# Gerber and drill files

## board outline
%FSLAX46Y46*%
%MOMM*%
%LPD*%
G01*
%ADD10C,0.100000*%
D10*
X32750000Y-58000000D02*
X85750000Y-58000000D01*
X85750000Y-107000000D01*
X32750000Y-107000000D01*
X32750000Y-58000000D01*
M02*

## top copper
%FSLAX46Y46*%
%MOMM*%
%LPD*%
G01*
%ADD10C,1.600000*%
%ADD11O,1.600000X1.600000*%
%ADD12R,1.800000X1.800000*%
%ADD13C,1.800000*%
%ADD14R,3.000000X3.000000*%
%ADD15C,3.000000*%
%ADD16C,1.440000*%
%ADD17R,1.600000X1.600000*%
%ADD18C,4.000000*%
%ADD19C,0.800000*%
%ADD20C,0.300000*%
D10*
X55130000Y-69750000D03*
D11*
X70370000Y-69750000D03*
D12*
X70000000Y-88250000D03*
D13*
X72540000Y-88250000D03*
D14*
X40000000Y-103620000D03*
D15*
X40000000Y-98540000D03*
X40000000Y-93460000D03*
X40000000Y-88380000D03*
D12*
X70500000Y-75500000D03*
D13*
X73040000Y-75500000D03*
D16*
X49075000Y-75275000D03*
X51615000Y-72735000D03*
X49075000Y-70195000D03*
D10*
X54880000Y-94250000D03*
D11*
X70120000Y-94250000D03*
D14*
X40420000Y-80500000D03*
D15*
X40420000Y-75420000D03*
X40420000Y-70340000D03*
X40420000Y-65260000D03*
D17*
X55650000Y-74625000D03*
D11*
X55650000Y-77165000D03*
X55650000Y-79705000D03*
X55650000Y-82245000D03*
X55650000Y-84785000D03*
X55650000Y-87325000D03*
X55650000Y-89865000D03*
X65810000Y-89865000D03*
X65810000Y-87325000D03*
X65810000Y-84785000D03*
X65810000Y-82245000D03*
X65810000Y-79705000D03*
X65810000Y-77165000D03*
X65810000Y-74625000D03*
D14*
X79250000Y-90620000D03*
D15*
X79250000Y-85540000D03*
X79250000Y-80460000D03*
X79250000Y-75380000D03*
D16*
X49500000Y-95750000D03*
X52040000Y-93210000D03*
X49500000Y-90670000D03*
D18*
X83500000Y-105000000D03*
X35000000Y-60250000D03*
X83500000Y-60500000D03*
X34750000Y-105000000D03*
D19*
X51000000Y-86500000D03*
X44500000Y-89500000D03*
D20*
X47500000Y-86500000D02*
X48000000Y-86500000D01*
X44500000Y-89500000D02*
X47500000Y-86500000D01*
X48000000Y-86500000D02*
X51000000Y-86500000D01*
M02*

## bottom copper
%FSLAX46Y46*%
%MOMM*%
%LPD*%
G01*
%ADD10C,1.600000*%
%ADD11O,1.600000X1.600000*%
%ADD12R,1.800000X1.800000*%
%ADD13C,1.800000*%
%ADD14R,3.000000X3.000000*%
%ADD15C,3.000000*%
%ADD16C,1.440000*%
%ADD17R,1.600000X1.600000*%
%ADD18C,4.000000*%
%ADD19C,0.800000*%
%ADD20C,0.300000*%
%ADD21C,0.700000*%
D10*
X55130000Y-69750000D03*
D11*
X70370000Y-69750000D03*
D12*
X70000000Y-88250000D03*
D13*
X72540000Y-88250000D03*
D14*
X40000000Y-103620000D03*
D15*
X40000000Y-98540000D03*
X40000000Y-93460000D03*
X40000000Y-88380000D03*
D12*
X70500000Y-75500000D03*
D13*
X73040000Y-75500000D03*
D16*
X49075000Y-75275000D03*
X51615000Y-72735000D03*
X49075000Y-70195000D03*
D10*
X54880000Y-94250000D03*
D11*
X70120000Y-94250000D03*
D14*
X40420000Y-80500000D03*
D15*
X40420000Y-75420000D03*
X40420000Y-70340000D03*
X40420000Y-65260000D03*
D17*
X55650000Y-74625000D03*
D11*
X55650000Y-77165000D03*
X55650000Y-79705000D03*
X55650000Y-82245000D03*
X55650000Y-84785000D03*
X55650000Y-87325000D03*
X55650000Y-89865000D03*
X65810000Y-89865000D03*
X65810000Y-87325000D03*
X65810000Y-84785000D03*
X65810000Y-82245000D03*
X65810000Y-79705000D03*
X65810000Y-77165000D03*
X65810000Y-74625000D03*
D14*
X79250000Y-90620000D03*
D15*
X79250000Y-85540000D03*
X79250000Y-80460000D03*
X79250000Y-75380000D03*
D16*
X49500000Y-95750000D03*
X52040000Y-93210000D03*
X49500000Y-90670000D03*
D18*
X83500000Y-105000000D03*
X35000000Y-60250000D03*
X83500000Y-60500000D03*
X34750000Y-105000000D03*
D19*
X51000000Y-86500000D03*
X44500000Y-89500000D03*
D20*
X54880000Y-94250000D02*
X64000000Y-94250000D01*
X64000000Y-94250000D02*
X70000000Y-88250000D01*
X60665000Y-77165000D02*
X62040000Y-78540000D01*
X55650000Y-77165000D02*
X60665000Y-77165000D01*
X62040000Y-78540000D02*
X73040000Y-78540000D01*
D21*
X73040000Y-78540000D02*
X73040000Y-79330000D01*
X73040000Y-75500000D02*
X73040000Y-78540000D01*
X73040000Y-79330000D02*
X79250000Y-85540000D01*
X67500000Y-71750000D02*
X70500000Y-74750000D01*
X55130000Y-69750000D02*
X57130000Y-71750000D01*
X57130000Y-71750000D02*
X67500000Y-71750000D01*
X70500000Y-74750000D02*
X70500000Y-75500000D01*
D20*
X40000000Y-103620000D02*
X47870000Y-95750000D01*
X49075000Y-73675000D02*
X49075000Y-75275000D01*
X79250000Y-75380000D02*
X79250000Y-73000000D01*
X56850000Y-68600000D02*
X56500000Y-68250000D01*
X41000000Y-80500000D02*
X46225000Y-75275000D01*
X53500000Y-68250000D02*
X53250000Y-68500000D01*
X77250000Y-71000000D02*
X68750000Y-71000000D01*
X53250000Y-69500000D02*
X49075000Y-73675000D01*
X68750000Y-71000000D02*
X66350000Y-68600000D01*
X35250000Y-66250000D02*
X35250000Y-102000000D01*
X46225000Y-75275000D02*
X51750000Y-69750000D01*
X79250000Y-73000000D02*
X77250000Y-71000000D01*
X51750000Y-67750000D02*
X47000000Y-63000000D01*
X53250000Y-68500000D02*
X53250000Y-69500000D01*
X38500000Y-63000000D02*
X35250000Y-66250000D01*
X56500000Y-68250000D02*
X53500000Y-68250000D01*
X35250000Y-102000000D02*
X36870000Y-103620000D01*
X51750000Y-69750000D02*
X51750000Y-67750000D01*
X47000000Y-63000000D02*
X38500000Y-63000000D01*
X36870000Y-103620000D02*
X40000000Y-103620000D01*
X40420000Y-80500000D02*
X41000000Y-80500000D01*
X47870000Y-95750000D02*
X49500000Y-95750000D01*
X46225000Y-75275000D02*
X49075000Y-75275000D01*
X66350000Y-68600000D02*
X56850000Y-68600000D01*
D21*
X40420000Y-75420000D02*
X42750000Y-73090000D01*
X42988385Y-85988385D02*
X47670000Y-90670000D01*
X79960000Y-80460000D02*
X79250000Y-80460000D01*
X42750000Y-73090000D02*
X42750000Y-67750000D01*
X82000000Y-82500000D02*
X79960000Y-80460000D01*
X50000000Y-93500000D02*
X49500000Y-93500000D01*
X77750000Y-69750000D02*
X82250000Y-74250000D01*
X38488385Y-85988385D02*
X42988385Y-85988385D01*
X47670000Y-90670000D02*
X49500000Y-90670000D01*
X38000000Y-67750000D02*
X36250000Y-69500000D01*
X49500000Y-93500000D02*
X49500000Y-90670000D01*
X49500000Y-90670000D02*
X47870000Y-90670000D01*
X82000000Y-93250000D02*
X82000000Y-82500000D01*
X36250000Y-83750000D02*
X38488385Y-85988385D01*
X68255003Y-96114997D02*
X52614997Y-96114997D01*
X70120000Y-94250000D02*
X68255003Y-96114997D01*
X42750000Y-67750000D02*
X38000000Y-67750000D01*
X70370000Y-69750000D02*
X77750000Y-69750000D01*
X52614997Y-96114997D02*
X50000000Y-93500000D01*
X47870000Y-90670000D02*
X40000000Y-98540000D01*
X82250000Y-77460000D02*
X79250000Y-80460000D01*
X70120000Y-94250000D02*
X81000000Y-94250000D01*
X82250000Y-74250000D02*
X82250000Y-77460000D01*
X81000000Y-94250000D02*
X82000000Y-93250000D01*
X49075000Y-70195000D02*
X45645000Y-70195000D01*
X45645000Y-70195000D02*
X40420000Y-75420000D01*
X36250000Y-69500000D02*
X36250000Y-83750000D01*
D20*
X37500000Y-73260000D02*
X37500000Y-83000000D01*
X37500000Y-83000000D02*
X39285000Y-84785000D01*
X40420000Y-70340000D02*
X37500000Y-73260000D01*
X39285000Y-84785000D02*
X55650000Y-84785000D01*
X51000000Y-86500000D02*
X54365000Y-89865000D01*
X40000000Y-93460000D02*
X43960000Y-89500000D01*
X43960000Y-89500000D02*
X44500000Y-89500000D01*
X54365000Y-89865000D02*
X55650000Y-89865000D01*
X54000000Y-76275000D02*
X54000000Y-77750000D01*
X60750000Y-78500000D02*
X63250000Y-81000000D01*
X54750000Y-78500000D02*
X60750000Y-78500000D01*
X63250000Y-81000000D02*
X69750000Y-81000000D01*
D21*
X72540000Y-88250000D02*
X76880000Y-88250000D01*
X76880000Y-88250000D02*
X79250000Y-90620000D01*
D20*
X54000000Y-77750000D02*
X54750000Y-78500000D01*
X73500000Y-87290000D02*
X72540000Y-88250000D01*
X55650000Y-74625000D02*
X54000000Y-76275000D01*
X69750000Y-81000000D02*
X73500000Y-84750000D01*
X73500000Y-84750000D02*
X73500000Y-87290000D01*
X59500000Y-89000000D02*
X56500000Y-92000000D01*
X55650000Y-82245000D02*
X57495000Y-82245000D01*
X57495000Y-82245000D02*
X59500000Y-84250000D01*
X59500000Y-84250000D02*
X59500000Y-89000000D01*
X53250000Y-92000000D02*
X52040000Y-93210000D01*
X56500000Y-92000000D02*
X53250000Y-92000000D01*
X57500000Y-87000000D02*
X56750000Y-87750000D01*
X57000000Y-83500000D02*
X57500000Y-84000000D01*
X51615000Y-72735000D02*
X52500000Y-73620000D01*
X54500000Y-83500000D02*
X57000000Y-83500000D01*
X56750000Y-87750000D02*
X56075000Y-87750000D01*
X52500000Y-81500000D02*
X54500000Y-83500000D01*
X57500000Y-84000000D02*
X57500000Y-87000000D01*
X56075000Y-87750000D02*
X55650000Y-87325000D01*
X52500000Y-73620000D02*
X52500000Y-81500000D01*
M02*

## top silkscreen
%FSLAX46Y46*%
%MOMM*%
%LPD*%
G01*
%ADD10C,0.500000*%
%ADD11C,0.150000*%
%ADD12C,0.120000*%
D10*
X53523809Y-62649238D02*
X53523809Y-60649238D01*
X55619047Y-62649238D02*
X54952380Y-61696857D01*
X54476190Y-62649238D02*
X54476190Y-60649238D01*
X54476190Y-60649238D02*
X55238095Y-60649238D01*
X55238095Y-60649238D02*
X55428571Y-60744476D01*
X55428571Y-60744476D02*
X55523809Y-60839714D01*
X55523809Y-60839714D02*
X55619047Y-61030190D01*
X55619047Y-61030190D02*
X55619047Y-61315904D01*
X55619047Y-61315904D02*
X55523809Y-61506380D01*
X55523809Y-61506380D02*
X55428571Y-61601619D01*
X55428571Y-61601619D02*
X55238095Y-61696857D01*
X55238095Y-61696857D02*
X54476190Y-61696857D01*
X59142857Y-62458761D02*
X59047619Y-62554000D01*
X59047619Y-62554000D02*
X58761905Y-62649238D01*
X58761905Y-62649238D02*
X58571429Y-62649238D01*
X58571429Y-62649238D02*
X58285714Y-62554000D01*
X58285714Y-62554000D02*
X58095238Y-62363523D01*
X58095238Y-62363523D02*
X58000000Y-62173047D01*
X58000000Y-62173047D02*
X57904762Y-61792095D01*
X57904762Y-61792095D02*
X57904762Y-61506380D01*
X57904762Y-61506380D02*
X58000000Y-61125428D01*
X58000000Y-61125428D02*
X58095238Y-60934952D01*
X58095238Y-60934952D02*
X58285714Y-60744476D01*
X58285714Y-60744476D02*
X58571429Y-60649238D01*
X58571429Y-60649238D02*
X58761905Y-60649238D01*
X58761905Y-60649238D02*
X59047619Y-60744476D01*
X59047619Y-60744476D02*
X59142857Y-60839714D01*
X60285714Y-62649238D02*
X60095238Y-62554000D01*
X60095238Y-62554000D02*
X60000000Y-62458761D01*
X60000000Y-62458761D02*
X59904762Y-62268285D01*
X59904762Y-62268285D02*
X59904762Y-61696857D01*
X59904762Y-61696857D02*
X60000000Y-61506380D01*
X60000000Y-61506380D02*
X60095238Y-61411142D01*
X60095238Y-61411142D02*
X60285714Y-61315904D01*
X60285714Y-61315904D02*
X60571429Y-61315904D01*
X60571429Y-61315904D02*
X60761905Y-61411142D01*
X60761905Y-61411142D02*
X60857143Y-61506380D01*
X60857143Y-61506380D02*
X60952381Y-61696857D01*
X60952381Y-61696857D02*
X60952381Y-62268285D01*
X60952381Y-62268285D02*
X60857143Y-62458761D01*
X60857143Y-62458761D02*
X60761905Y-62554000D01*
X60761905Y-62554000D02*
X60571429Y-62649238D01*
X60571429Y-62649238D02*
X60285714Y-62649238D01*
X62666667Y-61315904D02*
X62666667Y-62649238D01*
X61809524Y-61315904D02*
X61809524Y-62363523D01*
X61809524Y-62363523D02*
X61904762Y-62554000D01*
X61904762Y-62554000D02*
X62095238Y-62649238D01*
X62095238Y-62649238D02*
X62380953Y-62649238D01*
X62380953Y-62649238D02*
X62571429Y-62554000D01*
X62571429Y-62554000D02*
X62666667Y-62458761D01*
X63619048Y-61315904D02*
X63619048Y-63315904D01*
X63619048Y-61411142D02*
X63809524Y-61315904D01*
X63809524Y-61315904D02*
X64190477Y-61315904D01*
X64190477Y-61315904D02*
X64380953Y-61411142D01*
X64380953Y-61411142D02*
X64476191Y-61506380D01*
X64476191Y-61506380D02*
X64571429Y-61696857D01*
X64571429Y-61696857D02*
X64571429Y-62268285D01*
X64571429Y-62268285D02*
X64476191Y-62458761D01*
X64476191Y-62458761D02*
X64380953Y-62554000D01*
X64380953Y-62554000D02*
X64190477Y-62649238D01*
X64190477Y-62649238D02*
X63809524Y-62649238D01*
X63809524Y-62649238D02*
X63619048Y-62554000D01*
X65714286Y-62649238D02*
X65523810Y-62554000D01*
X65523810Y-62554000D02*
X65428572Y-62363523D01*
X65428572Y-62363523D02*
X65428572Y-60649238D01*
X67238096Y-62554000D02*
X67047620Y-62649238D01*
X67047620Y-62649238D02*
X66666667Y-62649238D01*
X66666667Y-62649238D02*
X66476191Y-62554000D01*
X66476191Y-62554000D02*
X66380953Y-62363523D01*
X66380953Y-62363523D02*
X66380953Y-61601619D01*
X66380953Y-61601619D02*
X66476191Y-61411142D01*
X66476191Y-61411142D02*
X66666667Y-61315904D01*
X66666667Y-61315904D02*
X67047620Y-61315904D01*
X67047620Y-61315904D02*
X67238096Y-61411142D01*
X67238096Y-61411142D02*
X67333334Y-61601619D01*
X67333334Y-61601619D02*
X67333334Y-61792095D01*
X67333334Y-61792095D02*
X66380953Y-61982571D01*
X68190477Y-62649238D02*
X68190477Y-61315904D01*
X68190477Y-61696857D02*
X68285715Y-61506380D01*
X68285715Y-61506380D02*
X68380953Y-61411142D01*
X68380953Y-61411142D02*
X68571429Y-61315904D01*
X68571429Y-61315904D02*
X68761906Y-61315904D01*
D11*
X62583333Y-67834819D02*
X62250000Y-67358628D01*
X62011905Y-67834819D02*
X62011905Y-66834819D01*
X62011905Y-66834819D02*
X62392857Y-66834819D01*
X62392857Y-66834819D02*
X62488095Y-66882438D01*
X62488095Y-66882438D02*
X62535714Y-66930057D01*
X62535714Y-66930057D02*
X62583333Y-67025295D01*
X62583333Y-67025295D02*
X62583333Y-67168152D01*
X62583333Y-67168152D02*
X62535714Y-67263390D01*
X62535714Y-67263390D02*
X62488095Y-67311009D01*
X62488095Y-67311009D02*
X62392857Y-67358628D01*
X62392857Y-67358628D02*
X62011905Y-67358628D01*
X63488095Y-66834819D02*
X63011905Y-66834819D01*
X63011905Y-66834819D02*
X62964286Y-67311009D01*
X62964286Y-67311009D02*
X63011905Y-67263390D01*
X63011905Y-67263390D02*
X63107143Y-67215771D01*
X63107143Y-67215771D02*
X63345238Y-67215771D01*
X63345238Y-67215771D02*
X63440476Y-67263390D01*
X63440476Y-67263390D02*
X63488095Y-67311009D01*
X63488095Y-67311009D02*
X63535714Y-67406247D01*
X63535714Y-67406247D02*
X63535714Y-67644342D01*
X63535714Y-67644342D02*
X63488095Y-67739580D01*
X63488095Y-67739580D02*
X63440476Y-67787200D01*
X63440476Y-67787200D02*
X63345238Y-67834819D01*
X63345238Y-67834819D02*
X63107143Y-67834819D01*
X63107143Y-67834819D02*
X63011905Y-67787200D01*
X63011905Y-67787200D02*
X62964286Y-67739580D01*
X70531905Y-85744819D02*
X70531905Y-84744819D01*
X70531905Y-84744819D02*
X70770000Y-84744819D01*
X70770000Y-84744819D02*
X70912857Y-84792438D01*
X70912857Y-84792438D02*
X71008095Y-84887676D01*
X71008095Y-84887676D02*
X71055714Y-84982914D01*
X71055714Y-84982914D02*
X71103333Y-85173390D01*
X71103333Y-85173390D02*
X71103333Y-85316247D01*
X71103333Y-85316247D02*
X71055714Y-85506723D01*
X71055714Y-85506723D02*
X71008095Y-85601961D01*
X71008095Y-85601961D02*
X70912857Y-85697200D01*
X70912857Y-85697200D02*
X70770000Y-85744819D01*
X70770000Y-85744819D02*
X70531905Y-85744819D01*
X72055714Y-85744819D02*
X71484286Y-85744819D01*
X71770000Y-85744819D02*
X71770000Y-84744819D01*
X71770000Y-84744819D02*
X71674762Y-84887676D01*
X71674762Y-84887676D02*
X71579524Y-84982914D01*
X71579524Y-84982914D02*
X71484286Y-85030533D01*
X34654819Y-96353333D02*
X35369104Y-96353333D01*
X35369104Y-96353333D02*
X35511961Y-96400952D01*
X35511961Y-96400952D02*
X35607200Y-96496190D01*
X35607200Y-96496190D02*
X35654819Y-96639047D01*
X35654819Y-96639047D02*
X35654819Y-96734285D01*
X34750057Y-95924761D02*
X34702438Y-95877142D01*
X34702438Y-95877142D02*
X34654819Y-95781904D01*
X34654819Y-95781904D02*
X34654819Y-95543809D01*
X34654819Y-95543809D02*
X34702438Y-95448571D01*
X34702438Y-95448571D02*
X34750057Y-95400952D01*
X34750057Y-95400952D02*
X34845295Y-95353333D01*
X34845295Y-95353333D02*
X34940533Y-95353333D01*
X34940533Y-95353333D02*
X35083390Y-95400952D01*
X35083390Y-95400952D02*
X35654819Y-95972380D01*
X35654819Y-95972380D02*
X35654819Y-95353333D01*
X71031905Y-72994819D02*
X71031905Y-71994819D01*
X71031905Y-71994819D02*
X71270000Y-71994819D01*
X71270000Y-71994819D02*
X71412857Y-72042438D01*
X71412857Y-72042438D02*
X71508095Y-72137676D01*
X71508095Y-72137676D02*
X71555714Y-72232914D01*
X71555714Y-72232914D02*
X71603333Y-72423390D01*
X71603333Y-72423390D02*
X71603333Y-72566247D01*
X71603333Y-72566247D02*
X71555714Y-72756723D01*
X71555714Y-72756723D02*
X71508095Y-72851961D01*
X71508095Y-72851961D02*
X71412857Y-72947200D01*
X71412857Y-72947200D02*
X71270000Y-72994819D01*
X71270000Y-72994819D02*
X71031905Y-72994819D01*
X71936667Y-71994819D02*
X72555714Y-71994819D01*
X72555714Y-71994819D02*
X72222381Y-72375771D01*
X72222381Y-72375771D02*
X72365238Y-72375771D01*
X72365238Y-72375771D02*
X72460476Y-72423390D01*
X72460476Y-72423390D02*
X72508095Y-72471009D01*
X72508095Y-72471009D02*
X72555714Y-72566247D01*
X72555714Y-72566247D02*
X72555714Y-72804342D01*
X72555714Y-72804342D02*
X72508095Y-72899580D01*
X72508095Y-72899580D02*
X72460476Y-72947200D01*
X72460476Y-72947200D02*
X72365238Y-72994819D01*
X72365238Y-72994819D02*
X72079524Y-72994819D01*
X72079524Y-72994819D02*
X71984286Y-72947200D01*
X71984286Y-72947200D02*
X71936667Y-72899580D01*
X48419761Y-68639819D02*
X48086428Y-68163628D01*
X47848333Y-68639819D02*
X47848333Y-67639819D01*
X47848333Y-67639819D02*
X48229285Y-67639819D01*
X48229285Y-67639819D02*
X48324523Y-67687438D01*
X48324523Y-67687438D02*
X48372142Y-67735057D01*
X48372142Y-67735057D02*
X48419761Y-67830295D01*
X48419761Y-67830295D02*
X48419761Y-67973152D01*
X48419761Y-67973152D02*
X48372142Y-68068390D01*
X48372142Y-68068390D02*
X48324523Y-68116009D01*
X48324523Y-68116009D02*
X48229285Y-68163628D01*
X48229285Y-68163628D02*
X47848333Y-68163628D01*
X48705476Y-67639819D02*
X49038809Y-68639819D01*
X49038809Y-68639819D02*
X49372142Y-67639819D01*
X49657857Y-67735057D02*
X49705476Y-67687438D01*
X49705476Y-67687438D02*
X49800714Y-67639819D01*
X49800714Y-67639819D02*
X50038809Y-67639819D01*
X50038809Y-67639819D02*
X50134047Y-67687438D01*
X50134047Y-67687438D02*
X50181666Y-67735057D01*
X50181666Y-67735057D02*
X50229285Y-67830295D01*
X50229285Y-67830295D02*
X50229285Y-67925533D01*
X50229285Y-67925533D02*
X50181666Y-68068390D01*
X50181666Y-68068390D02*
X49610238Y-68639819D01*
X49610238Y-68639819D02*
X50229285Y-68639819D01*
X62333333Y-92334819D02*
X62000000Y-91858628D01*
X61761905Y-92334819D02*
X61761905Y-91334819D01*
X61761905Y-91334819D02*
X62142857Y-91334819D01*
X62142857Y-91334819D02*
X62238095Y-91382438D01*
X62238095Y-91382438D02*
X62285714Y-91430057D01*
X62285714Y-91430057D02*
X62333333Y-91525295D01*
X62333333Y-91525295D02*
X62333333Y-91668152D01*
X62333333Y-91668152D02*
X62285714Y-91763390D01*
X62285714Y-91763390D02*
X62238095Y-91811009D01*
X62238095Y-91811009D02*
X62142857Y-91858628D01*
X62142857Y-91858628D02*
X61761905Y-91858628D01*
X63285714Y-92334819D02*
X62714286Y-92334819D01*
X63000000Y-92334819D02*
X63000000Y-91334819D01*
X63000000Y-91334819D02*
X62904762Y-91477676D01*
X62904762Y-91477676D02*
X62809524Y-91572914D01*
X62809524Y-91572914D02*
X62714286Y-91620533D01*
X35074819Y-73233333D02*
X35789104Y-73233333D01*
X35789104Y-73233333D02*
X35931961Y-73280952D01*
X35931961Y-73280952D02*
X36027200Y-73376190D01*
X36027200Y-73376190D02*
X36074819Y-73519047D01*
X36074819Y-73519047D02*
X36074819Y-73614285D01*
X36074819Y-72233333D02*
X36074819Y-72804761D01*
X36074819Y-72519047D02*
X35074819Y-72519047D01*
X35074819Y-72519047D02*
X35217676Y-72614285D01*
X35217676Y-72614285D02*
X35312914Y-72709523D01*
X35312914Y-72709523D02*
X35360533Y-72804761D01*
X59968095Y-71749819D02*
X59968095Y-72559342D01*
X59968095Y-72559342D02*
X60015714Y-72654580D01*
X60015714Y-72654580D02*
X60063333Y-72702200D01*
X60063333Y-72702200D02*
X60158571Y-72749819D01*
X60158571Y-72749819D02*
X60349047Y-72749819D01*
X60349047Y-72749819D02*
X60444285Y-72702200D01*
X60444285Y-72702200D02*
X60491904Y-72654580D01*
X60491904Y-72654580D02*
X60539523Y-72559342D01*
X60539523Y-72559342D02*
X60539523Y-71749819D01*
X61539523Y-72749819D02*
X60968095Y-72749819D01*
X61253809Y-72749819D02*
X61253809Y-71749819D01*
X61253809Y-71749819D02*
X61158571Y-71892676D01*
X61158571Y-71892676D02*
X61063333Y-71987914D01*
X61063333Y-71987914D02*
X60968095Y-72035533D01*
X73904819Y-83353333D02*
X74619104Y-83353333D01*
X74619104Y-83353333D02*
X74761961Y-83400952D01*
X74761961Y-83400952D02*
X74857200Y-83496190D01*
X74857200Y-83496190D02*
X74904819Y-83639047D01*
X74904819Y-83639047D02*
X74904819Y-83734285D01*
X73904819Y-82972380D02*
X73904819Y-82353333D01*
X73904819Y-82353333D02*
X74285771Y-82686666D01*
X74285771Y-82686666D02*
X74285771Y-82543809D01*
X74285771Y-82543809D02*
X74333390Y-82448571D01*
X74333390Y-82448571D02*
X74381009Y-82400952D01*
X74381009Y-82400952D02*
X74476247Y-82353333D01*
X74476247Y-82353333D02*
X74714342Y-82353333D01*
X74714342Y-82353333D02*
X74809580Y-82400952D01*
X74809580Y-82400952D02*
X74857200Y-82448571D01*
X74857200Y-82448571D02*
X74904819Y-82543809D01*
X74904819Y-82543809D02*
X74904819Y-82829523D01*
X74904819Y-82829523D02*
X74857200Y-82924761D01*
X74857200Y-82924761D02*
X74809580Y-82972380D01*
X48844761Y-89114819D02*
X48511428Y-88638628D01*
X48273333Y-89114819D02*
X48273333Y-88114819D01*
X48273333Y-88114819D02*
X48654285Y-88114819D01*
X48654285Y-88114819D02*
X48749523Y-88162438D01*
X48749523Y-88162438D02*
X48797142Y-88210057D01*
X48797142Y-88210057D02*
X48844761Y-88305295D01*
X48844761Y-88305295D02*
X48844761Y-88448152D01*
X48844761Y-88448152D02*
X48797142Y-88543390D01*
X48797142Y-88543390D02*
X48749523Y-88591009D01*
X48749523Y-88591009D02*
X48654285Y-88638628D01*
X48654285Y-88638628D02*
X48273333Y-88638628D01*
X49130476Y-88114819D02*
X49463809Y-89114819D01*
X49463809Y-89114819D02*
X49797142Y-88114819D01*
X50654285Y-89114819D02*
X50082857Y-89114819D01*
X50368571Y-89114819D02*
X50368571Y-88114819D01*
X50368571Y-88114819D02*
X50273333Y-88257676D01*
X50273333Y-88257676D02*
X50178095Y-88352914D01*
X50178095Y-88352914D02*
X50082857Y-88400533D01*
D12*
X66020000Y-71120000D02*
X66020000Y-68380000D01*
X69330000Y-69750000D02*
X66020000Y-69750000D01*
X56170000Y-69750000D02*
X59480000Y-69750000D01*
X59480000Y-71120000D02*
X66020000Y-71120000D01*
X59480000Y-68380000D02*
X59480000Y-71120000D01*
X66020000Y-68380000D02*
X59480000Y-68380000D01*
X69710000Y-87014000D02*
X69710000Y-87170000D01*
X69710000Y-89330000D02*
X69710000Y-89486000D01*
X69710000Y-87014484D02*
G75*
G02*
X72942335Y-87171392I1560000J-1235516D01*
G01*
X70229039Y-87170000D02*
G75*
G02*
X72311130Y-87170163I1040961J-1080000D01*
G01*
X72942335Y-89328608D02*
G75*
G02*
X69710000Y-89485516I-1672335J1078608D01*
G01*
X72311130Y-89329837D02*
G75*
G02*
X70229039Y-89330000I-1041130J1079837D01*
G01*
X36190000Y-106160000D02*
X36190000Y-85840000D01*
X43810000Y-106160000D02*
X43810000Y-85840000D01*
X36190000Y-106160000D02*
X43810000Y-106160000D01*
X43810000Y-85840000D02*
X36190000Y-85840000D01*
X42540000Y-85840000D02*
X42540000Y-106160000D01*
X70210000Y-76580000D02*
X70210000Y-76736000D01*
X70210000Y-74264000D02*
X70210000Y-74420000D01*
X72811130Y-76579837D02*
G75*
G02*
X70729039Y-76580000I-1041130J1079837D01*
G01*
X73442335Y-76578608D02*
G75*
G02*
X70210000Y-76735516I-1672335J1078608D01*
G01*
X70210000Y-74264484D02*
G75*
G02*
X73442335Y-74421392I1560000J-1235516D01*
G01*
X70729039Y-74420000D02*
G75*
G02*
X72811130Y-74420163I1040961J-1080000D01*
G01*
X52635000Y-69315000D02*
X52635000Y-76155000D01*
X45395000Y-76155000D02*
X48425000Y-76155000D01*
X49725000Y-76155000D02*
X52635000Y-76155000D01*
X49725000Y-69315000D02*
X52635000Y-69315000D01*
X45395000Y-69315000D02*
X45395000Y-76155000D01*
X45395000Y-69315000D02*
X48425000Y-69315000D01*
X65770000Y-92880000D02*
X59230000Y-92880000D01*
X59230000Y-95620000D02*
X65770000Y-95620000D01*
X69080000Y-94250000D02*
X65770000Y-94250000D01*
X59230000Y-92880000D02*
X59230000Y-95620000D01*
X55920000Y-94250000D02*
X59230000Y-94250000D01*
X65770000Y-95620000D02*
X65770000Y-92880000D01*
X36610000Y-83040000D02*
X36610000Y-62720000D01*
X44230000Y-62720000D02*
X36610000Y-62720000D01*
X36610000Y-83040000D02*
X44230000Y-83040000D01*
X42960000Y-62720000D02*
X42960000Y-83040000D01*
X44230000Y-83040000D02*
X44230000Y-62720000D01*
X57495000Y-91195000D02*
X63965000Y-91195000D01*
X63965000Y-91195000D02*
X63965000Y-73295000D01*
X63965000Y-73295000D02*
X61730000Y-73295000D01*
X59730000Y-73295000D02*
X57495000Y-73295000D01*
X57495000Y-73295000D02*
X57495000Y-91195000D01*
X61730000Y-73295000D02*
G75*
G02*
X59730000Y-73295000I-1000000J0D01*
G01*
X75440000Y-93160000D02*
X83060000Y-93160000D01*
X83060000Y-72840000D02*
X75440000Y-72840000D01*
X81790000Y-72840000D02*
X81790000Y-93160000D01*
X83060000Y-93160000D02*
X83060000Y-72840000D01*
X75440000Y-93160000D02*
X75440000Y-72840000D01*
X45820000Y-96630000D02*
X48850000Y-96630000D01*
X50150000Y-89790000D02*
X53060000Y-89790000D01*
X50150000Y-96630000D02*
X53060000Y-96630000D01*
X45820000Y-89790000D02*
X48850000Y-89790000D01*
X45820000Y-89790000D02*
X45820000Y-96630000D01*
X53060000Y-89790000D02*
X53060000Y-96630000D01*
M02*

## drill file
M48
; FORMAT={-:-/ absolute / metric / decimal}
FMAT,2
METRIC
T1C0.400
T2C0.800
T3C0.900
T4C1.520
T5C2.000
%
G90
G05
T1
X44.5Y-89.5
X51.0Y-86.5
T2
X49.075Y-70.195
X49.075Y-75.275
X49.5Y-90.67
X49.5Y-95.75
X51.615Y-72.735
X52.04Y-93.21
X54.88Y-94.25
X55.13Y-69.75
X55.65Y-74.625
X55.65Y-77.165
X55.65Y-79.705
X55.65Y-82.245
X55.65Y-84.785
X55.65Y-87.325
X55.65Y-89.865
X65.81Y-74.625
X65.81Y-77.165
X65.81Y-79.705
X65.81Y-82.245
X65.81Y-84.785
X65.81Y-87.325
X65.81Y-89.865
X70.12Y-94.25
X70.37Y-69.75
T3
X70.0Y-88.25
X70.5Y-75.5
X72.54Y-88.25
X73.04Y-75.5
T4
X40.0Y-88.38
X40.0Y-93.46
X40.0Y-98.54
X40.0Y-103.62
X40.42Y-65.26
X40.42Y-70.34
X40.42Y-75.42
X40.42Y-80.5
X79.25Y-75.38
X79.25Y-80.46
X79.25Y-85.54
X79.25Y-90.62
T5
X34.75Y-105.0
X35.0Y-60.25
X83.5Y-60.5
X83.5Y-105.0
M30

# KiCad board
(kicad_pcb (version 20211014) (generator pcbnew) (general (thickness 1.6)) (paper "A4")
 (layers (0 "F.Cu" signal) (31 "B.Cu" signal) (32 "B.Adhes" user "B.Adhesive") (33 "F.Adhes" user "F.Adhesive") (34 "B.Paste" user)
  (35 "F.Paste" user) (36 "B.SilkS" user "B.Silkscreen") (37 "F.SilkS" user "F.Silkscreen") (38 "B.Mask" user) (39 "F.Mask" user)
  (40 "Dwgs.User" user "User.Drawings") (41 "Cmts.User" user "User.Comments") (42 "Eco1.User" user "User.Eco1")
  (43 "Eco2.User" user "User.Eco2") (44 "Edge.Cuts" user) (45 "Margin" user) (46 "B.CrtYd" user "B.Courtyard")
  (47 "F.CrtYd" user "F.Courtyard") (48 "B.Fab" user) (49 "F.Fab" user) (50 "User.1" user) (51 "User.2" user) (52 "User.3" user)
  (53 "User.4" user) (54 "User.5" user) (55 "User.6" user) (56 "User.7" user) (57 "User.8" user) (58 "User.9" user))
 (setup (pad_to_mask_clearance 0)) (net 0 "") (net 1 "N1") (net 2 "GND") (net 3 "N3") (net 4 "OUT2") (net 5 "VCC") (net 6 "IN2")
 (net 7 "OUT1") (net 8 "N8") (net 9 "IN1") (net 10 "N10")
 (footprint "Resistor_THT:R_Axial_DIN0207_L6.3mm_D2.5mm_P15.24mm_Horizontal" (layer "F.Cu") (at 55.13 69.75)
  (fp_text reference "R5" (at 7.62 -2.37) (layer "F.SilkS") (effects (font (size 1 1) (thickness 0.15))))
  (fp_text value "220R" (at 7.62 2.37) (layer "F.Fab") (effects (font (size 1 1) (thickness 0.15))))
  (fp_line (start 10.89 1.37) (end 10.89 -1.37) (layer "F.SilkS") (width 0.12))
  (fp_line (start 14.2 0) (end 10.89 0) (layer "F.SilkS") (width 0.12))
  (fp_line (start 1.04 0) (end 4.35 0) (layer "F.SilkS") (width 0.12))
  (fp_line (start 4.35 1.37) (end 10.89 1.37) (layer "F.SilkS") (width 0.12))
  (fp_line (start 4.35 -1.37) (end 4.35 1.37) (layer "F.SilkS") (width 0.12))
  (fp_line (start 10.89 -1.37) (end 4.35 -1.37) (layer "F.SilkS") (width 0.12))
  (pad "1" thru_hole circle (at 0 0) (size 1.6 1.6) (drill 0.8) (layers *.Cu *.Mask) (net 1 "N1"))
  (pad "2" thru_hole oval (at 15.24 0) (size 1.6 1.6) (drill 0.8) (layers *.Cu *.Mask) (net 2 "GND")))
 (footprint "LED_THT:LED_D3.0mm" (layer "F.Cu") (at 70 88.25)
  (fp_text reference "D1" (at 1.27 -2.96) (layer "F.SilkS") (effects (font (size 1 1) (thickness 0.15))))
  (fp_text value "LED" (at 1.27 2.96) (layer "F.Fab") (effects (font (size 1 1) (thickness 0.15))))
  (fp_line (start -0.29 -1.236) (end -0.29 -1.08) (layer "F.SilkS") (width 0.12))
  (fp_line (start -0.29 1.08) (end -0.29 1.236) (layer "F.SilkS") (width 0.12))
  (fp_arc (start -0.29 -1.235516) (mid 1.366487 -1.987659) (end 2.942335 -1.078608) (layer "F.SilkS") (width 0.12))
  (fp_arc (start 0.229039 -1.08) (mid 1.270117 -1.5) (end 2.31113 -1.079837) (layer "F.SilkS") (width 0.12))
  (fp_arc (start 2.942335 1.078608) (mid 1.366487 1.987659) (end -0.29 1.235516) (layer "F.SilkS") (width 0.12))
  (fp_arc (start 2.31113 1.079837) (mid 1.270117 1.5) (end 0.229039 1.08) (layer "F.SilkS") (width 0.12))
  (pad "1" thru_hole rect (at 0 0) (size 1.8 1.8) (drill 0.9) (layers *.Cu *.Mask) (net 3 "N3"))
  (pad "2" thru_hole circle (at 2.54 0) (size 1.8 1.8) (drill 0.9) (layers *.Cu *.Mask) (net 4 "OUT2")))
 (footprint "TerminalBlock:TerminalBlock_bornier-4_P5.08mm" (layer "F.Cu") (at 40 103.62 90)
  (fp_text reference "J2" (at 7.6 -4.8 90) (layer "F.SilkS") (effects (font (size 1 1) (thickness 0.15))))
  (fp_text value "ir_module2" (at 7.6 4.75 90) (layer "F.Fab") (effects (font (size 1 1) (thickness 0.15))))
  (fp_line (start -2.54 -3.81) (end 17.78 -3.81) (layer "F.SilkS") (width 0.12))
  (fp_line (start -2.54 3.81) (end 17.78 3.81) (layer "F.SilkS") (width 0.12))
  (fp_line (start -2.54 -3.81) (end -2.54 3.81) (layer "F.SilkS") (width 0.12))
  (fp_line (start 17.78 3.81) (end 17.78 -3.81) (layer "F.SilkS") (width 0.12))
  (fp_line (start 17.78 2.54) (end -2.54 2.54) (layer "F.SilkS") (width 0.12))
  (pad "1" thru_hole rect (at 0 0 90) (size 3 3) (drill 1.52) (layers *.Cu *.Mask) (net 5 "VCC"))
  (pad "2" thru_hole circle (at 5.08 0 90) (size 3 3) (drill 1.52) (layers *.Cu *.Mask) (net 2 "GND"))
  (pad "3" thru_hole circle (at 10.16 0 90) (size 3 3) (drill 1.52) (layers *.Cu *.Mask) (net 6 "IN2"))
  (pad "4" thru_hole circle (at 15.24 0 90) (size 3 3) (drill 1.52) (layers *.Cu *.Mask)))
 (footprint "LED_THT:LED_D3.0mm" (layer "F.Cu") (at 70.5 75.5)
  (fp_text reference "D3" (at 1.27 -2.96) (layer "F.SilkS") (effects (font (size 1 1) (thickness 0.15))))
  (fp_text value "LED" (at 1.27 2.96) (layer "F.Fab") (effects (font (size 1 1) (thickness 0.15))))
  (fp_line (start -0.29 1.08) (end -0.29 1.236) (layer "F.SilkS") (width 0.12))
  (fp_line (start -0.29 -1.236) (end -0.29 -1.08) (layer "F.SilkS") (width 0.12))
  (fp_arc (start 2.31113 1.079837) (mid 1.270117 1.5) (end 0.229039 1.08) (layer "F.SilkS") (width 0.12))
  (fp_arc (start 2.942335 1.078608) (mid 1.366487 1.987659) (end -0.29 1.235516) (layer "F.SilkS") (width 0.12))
  (fp_arc (start -0.29 -1.235516) (mid 1.366487 -1.987659) (end 2.942335 -1.078608) (layer "F.SilkS") (width 0.12))
  (fp_arc (start 0.229039 -1.08) (mid 1.270117 -1.5) (end 2.31113 -1.079837) (layer "F.SilkS") (width 0.12))
  (pad "1" thru_hole rect (at 0 0) (size 1.8 1.8) (drill 0.9) (layers *.Cu *.Mask) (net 1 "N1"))
  (pad "2" thru_hole circle (at 2.54 0) (size 1.8 1.8) (drill 0.9) (layers *.Cu *.Mask) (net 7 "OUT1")))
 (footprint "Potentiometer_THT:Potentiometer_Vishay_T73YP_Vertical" (layer "F.Cu") (at 49.075 75.275)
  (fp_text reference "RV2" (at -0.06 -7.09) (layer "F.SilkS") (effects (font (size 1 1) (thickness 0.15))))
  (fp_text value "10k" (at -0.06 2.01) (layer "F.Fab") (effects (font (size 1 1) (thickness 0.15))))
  (fp_line (start 3.56 -5.96) (end 3.56 0.88) (layer "F.SilkS") (width 0.12))
  (fp_line (start -3.68 0.88) (end -0.65 0.88) (layer "F.SilkS") (width 0.12))
  (fp_line (start 0.65 0.88) (end 3.56 0.88) (layer "F.SilkS") (width 0.12))
  (fp_line (start 0.65 -5.96) (end 3.56 -5.96) (layer "F.SilkS") (width 0.12))
  (fp_line (start -3.68 -5.96) (end -3.68 0.88) (layer "F.SilkS") (width 0.12))
  (fp_line (start -3.68 -5.96) (end -0.65 -5.96) (layer "F.SilkS") (width 0.12))
  (pad "1" thru_hole circle (at 0 0) (size 1.44 1.44) (drill 0.8) (layers *.Cu *.Mask) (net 5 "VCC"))
  (pad "2" thru_hole circle (at 2.54 -2.54) (size 1.44 1.44) (drill 0.8) (layers *.Cu *.Mask) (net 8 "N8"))
  (pad "3" thru_hole circle (at 0 -5.08) (size 1.44 1.44) (drill 0.8) (layers *.Cu *.Mask) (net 2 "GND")))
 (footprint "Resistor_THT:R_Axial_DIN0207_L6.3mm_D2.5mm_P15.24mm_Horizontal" (layer "F.Cu") (at 54.88 94.25)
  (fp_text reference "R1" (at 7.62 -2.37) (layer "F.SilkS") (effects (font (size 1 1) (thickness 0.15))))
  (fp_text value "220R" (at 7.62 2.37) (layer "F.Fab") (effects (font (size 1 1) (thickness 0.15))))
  (fp_line (start 10.89 -1.37) (end 4.35 -1.37) (layer "F.SilkS") (width 0.12))
  (fp_line (start 4.35 1.37) (end 10.89 1.37) (layer "F.SilkS") (width 0.12))
  (fp_line (start 14.2 0) (end 10.89 0) (layer "F.SilkS") (width 0.12))
  (fp_line (start 4.35 -1.37) (end 4.35 1.37) (layer "F.SilkS") (width 0.12))
  (fp_line (start 1.04 0) (end 4.35 0) (layer "F.SilkS") (width 0.12))
  (fp_line (start 10.89 1.37) (end 10.89 -1.37) (layer "F.SilkS") (width 0.12))
  (pad "1" thru_hole circle (at 0 0) (size 1.6 1.6) (drill 0.8) (layers *.Cu *.Mask) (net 3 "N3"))
  (pad "2" thru_hole oval (at 15.24 0) (size 1.6 1.6) (drill 0.8) (layers *.Cu *.Mask) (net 2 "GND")))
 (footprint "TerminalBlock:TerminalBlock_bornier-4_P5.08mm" (layer "F.Cu") (at 40.42 80.5 90)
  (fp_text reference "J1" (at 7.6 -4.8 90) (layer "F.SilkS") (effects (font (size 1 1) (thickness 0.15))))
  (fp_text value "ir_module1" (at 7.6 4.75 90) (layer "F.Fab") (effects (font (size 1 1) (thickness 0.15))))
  (fp_line (start -2.54 -3.81) (end 17.78 -3.81) (layer "F.SilkS") (width 0.12))
  (fp_line (start 17.78 3.81) (end 17.78 -3.81) (layer "F.SilkS") (width 0.12))
  (fp_line (start -2.54 -3.81) (end -2.54 3.81) (layer "F.SilkS") (width 0.12))
  (fp_line (start 17.78 2.54) (end -2.54 2.54) (layer "F.SilkS") (width 0.12))
  (fp_line (start -2.54 3.81) (end 17.78 3.81) (layer "F.SilkS") (width 0.12))
  (pad "1" thru_hole rect (at 0 0 90) (size 3 3) (drill 1.52) (layers *.Cu *.Mask) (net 5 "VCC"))
  (pad "2" thru_hole circle (at 5.08 0 90) (size 3 3) (drill 1.52) (layers *.Cu *.Mask) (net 2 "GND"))
  (pad "3" thru_hole circle (at 10.16 0 90) (size 3 3) (drill 1.52) (layers *.Cu *.Mask) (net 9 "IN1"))
  (pad "4" thru_hole circle (at 15.24 0 90) (size 3 3) (drill 1.52) (layers *.Cu *.Mask)))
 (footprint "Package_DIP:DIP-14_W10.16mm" (layer "F.Cu") (at 55.65 74.625)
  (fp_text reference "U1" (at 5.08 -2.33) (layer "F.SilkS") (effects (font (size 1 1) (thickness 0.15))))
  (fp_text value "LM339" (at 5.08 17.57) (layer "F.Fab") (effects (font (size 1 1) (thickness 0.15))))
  (fp_line (start 1.845 16.57) (end 8.315 16.57) (layer "F.SilkS") (width 0.12))
  (fp_line (start 8.315 16.57) (end 8.315 -1.33) (layer "F.SilkS") (width 0.12))
  (fp_line (start 8.315 -1.33) (end 6.08 -1.33) (layer "F.SilkS") (width 0.12))
  (fp_line (start 4.08 -1.33) (end 1.845 -1.33) (layer "F.SilkS") (width 0.12))
  (fp_line (start 1.845 -1.33) (end 1.845 16.57) (layer "F.SilkS") (width 0.12))
  (fp_arc (start 6.08 -1.33) (mid 5.08 -0.33) (end 4.08 -1.33) (layer "F.SilkS") (width 0.12))
  (pad "1" thru_hole rect (at 0 0) (size 1.6 1.6) (drill 0.8) (layers *.Cu *.Mask) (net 4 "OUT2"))
  (pad "2" thru_hole oval (at 0 2.54) (size 1.6 1.6) (drill 0.8) (layers *.Cu *.Mask) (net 7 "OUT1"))
  (pad "3" thru_hole oval (at 0 5.08) (size 1.6 1.6) (drill 0.8) (layers *.Cu *.Mask))
  (pad "4" thru_hole oval (at 0 7.62) (size 1.6 1.6) (drill 0.8) (layers *.Cu *.Mask) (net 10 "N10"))
  (pad "5" thru_hole oval (at 0 10.16) (size 1.6 1.6) (drill 0.8) (layers *.Cu *.Mask) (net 9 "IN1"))
  (pad "6" thru_hole oval (at 0 12.7) (size 1.6 1.6) (drill 0.8) (layers *.Cu *.Mask) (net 8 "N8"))
  (pad "7" thru_hole oval (at 0 15.24) (size 1.6 1.6) (drill 0.8) (layers *.Cu *.Mask) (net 6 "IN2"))
  (pad "8" thru_hole oval (at 10.16 15.24) (size 1.6 1.6) (drill 0.8) (layers *.Cu *.Mask))
  (pad "9" thru_hole oval (at 10.16 12.7) (size 1.6 1.6) (drill 0.8) (layers *.Cu *.Mask))
  (pad "10" thru_hole oval (at 10.16 10.16) (size 1.6 1.6) (drill 0.8) (layers *.Cu *.Mask))
  (pad "11" thru_hole oval (at 10.16 7.62) (size 1.6 1.6) (drill 0.8) (layers *.Cu *.Mask))
  (pad "12" thru_hole oval (at 10.16 5.08) (size 1.6 1.6) (drill 0.8) (layers *.Cu *.Mask))
  (pad "13" thru_hole oval (at 10.16 2.54) (size 1.6 1.6) (drill 0.8) (layers *.Cu *.Mask))
  (pad "14" thru_hole oval (at 10.16 0) (size 1.6 1.6) (drill 0.8) (layers *.Cu *.Mask)))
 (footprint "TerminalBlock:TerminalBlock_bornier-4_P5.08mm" (layer "F.Cu") (at 79.25 90.62 90)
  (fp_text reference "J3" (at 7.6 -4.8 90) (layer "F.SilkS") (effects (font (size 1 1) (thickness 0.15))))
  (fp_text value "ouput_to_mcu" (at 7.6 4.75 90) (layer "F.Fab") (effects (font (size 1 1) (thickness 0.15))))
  (fp_line (start -2.54 -3.81) (end -2.54 3.81) (layer "F.SilkS") (width 0.12))
  (fp_line (start 17.78 3.81) (end 17.78 -3.81) (layer "F.SilkS") (width 0.12))
  (fp_line (start 17.78 2.54) (end -2.54 2.54) (layer "F.SilkS") (width 0.12))
  (fp_line (start -2.54 3.81) (end 17.78 3.81) (layer "F.SilkS") (width 0.12))
  (fp_line (start -2.54 -3.81) (end 17.78 -3.81) (layer "F.SilkS") (width 0.12))
  (pad "1" thru_hole rect (at 0 0 90) (size 3 3) (drill 1.52) (layers *.Cu *.Mask) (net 4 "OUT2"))
  (pad "2" thru_hole circle (at 5.08 0 90) (size 3 3) (drill 1.52) (layers *.Cu *.Mask) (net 7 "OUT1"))
  (pad "3" thru_hole circle (at 10.16 0 90) (size 3 3) (drill 1.52) (layers *.Cu *.Mask) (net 2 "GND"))
  (pad "4" thru_hole circle (at 15.24 0 90) (size 3 3) (drill 1.52) (layers *.Cu *.Mask) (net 5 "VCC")))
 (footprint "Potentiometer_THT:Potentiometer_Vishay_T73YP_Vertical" (layer "F.Cu") (at 49.5 95.75)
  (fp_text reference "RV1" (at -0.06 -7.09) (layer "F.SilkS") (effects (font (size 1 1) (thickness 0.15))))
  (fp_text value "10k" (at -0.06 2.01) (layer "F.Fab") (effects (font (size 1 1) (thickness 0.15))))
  (fp_line (start -3.68 0.88) (end -0.65 0.88) (layer "F.SilkS") (width 0.12))
  (fp_line (start 0.65 -5.96) (end 3.56 -5.96) (layer "F.SilkS") (width 0.12))
  (fp_line (start 0.65 0.88) (end 3.56 0.88) (layer "F.SilkS") (width 0.12))
  (fp_line (start -3.68 -5.96) (end -0.65 -5.96) (layer "F.SilkS") (width 0.12))
  (fp_line (start -3.68 -5.96) (end -3.68 0.88) (layer "F.SilkS") (width 0.12))
  (fp_line (start 3.56 -5.96) (end 3.56 0.88) (layer "F.SilkS") (width 0.12))
  (pad "1" thru_hole circle (at 0 0) (size 1.44 1.44) (drill 0.8) (layers *.Cu *.Mask) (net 5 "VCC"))
  (pad "2" thru_hole circle (at 2.54 -2.54) (size 1.44 1.44) (drill 0.8) (layers *.Cu *.Mask) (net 10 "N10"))
  (pad "3" thru_hole circle (at 0 -5.08) (size 1.44 1.44) (drill 0.8) (layers *.Cu *.Mask) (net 2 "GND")))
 (gr_rect (start 32.75 58) (end 85.75 107) (layer "Edge.Cuts") (width 0.1) (fill none))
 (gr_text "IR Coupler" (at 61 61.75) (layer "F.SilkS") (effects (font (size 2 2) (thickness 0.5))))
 (via (at 83.5 105) (size 4) (drill 2) (layers "F.Cu" "B.Cu") (free) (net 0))
 (via (at 35 60.25) (size 4) (drill 2) (layers "F.Cu" "B.Cu") (free) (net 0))
 (via (at 83.5 60.5) (size 4) (drill 2) (layers "F.Cu" "B.Cu") (free) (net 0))
 (via (at 34.75 105) (size 4) (drill 2) (layers "F.Cu" "B.Cu") (free) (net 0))
 (segment (start 54.88 94.25) (end 64 94.25) (width 0.3) (layer "B.Cu") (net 3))
 (segment (start 64 94.25) (end 70 88.25) (width 0.3) (layer "B.Cu") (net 3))
 (segment (start 60.665 77.165) (end 62.04 78.54) (width 0.3) (layer "B.Cu") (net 7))
 (segment (start 55.65 77.165) (end 60.665 77.165) (width 0.3) (layer "B.Cu") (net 7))
 (segment (start 62.04 78.54) (end 73.04 78.54) (width 0.3) (layer "B.Cu") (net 7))
 (segment (start 73.04 78.54) (end 73.04 79.33) (width 0.7) (layer "B.Cu") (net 7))
 (segment (start 73.04 75.5) (end 73.04 78.54) (width 0.7) (layer "B.Cu") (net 7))
 (segment (start 73.04 79.33) (end 79.25 85.54) (width 0.7) (layer "B.Cu") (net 7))
 (segment (start 67.5 71.75) (end 70.5 74.75) (width 0.7) (layer "B.Cu") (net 1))
 (segment (start 55.13 69.75) (end 57.13 71.75) (width 0.7) (layer "B.Cu") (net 1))
 (segment (start 57.13 71.75) (end 67.5 71.75) (width 0.7) (layer "B.Cu") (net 1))
 (segment (start 70.5 74.75) (end 70.5 75.5) (width 0.7) (layer "B.Cu") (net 1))
 (segment (start 40 103.62) (end 47.87 95.75) (width 0.3) (layer "B.Cu") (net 5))
 (segment (start 49.075 73.675) (end 49.075 75.275) (width 0.3) (layer "B.Cu") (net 5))
 (segment (start 79.25 75.38) (end 79.25 73) (width 0.3) (layer "B.Cu") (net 5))
 (segment (start 56.85 68.6) (end 56.5 68.25) (width 0.3) (layer "B.Cu") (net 5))
 (segment (start 41 80.5) (end 46.225 75.275) (width 0.3) (layer "B.Cu") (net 5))
 (segment (start 53.5 68.25) (end 53.25 68.5) (width 0.3) (layer "B.Cu") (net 5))
 (segment (start 77.25 71) (end 68.75 71) (width 0.3) (layer "B.Cu") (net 5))
 (segment (start 53.25 69.5) (end 49.075 73.675) (width 0.3) (layer "B.Cu") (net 5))
 (segment (start 68.75 71) (end 66.35 68.6) (width 0.3) (layer "B.Cu") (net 5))
 (segment (start 35.25 66.25) (end 35.25 102) (width 0.3) (layer "B.Cu") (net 5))
 (segment (start 46.225 75.275) (end 51.75 69.75) (width 0.3) (layer "B.Cu") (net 5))
 (segment (start 79.25 73) (end 77.25 71) (width 0.3) (layer "B.Cu") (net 5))
 (segment (start 51.75 67.75) (end 47 63) (width 0.3) (layer "B.Cu") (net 5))
 (segment (start 53.25 68.5) (end 53.25 69.5) (width 0.3) (layer "B.Cu") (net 5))
 (segment (start 38.5 63) (end 35.25 66.25) (width 0.3) (layer "B.Cu") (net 5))
 (segment (start 56.5 68.25) (end 53.5 68.25) (width 0.3) (layer "B.Cu") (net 5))
 (segment (start 35.25 102) (end 36.87 103.62) (width 0.3) (layer "B.Cu") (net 5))
 (segment (start 51.75 69.75) (end 51.75 67.75) (width 0.3) (layer "B.Cu") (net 5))
 (segment (start 47 63) (end 38.5 63) (width 0.3) (layer "B.Cu") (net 5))
 (segment (start 36.87 103.62) (end 40 103.62) (width 0.3) (layer "B.Cu") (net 5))
 (segment (start 40.42 80.5) (end 41 80.5) (width 0.3) (layer "B.Cu") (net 5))
 (segment (start 47.87 95.75) (end 49.5 95.75) (width 0.3) (layer "B.Cu") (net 5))
 (segment (start 46.225 75.275) (end 49.075 75.275) (width 0.3) (layer "B.Cu") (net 5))
 (segment (start 66.35 68.6) (end 56.85 68.6) (width 0.3) (layer "B.Cu") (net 5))
 (segment (start 40.42 75.42) (end 42.75 73.09) (width 0.7) (layer "B.Cu") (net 2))
 (segment (start 42.988385 85.988385) (end 47.67 90.67) (width 0.7) (layer "B.Cu") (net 2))
 (segment (start 79.96 80.46) (end 79.25 80.46) (width 0.7) (layer "B.Cu") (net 2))
 (segment (start 42.75 73.09) (end 42.75 67.75) (width 0.7) (layer "B.Cu") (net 2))
 (segment (start 82 82.5) (end 79.96 80.46) (width 0.7) (layer "B.Cu") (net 2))
 (segment (start 50 93.5) (end 49.5 93.5) (width 0.7) (layer "B.Cu") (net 2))
 (segment (start 77.75 69.75) (end 82.25 74.25) (width 0.7) (layer "B.Cu") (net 2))
 (segment (start 38.488385 85.988385) (end 42.988385 85.988385) (width 0.7) (layer "B.Cu") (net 2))
 (segment (start 47.67 90.67) (end 49.5 90.67) (width 0.7) (layer "B.Cu") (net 2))
 (segment (start 38 67.75) (end 36.25 69.5) (width 0.7) (layer "B.Cu") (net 2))
 (segment (start 49.5 93.5) (end 49.5 90.67) (width 0.7) (layer "B.Cu") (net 2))
 (segment (start 49.5 90.67) (end 47.87 90.67) (width 0.7) (layer "B.Cu") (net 2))
 (segment (start 82 93.25) (end 82 82.5) (width 0.7) (layer "B.Cu") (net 2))
 (segment (start 36.25 83.75) (end 38.488385 85.988385) (width 0.7) (layer "B.Cu") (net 2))
 (segment (start 68.255003 96.114997) (end 52.614997 96.114997) (width 0.7) (layer "B.Cu") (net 2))
 (segment (start 70.12 94.25) (end 68.255003 96.114997) (width 0.7) (layer "B.Cu") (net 2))
 (segment (start 42.75 67.75) (end 38 67.75) (width 0.7) (layer "B.Cu") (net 2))
 (segment (start 70.37 69.75) (end 77.75 69.75) (width 0.7) (layer "B.Cu") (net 2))
 (segment (start 52.614997 96.114997) (end 50 93.5) (width 0.7) (layer "B.Cu") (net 2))
 (segment (start 47.87 90.67) (end 40 98.54) (width 0.7) (layer "B.Cu") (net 2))
 (segment (start 82.25 77.46) (end 79.25 80.46) (width 0.7) (layer "B.Cu") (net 2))
 (segment (start 70.12 94.25) (end 81 94.25) (width 0.7) (layer "B.Cu") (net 2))
 (segment (start 82.25 74.25) (end 82.25 77.46) (width 0.7) (layer "B.Cu") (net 2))
 (segment (start 81 94.25) (end 82 93.25) (width 0.7) (layer "B.Cu") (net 2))
 (segment (start 49.075 70.195) (end 45.645 70.195) (width 0.7) (layer "B.Cu") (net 2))
 (segment (start 45.645 70.195) (end 40.42 75.42) (width 0.7) (layer "B.Cu") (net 2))
 (segment (start 36.25 69.5) (end 36.25 83.75) (width 0.7) (layer "B.Cu") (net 2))
 (segment (start 37.5 73.26) (end 37.5 83) (width 0.3) (layer "B.Cu") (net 9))
 (segment (start 37.5 83) (end 39.285 84.785) (width 0.3) (layer "B.Cu") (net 9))
 (segment (start 40.42 70.34) (end 37.5 73.26) (width 0.3) (layer "B.Cu") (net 9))
 (segment (start 39.285 84.785) (end 55.65 84.785) (width 0.3) (layer "B.Cu") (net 9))
 (segment (start 47.5 86.5) (end 48 86.5) (width 0.3) (layer "F.Cu") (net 6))
 (segment (start 44.5 89.5) (end 47.5 86.5) (width 0.3) (layer "F.Cu") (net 6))
 (segment (start 48 86.5) (end 51 86.5) (width 0.3) (layer "F.Cu") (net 6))
 (via (at 51 86.5) (size 0.8) (drill 0.4) (layers "F.Cu" "B.Cu") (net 6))
 (via (at 44.5 89.5) (size 0.8) (drill 0.4) (layers "F.Cu" "B.Cu") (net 6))
 (segment (start 51 86.5) (end 54.365 89.865) (width 0.3) (layer "B.Cu") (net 6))
 (segment (start 40 93.46) (end 43.96 89.5) (width 0.3) (layer "B.Cu") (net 6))
 (segment (start 43.96 89.5) (end 44.5 89.5) (width 0.3) (layer "B.Cu") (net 6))
 (segment (start 54.365 89.865) (end 55.65 89.865) (width 0.3) (layer "B.Cu") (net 6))
 (segment (start 54 76.275) (end 54 77.75) (width 0.3) (layer "B.Cu") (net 4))
 (segment (start 60.75 78.5) (end 63.25 81) (width 0.3) (layer "B.Cu") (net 4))
 (segment (start 54.75 78.5) (end 60.75 78.5) (width 0.3) (layer "B.Cu") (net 4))
 (segment (start 63.25 81) (end 69.75 81) (width 0.3) (layer "B.Cu") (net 4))
 (segment (start 72.54 88.25) (end 76.88 88.25) (width 0.7) (layer "B.Cu") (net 4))
 (segment (start 76.88 88.25) (end 79.25 90.62) (width 0.7) (layer "B.Cu") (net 4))
 (segment (start 54 77.75) (end 54.75 78.5) (width 0.3) (layer "B.Cu") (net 4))
 (segment (start 73.5 87.29) (end 72.54 88.25) (width 0.3) (layer "B.Cu") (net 4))
 (segment (start 55.65 74.625) (end 54 76.275) (width 0.3) (layer "B.Cu") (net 4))
 (segment (start 69.75 81) (end 73.5 84.75) (width 0.3) (layer "B.Cu") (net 4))
 (segment (start 73.5 84.75) (end 73.5 87.29) (width 0.3) (layer "B.Cu") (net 4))
 (segment (start 59.5 89) (end 56.5 92) (width 0.3) (layer "B.Cu") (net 10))
 (segment (start 55.65 82.245) (end 57.495 82.245) (width 0.3) (layer "B.Cu") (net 10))
 (segment (start 57.495 82.245) (end 59.5 84.25) (width 0.3) (layer "B.Cu") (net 10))
 (segment (start 59.5 84.25) (end 59.5 89) (width 0.3) (layer "B.Cu") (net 10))
 (segment (start 53.25 92) (end 52.04 93.21) (width 0.3) (layer "B.Cu") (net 10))
 (segment (start 56.5 92) (end 53.25 92) (width 0.3) (layer "B.Cu") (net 10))
 (segment (start 57.5 87) (end 56.75 87.75) (width 0.3) (layer "B.Cu") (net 8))
 (segment (start 57 83.5) (end 57.5 84) (width 0.3) (layer "B.Cu") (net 8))
 (segment (start 51.615 72.735) (end 52.5 73.62) (width 0.3) (layer "B.Cu") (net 8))
 (segment (start 54.5 83.5) (end 57 83.5) (width 0.3) (layer "B.Cu") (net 8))
 (segment (start 56.75 87.75) (end 56.075 87.75) (width 0.3) (layer "B.Cu") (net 8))
 (segment (start 52.5 81.5) (end 54.5 83.5) (width 0.3) (layer "B.Cu") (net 8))
 (segment (start 57.5 84) (end 57.5 87) (width 0.3) (layer "B.Cu") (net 8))
 (segment (start 56.075 87.75) (end 55.65 87.325) (width 0.3) (layer "B.Cu") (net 8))
 (segment (start 52.5 73.62) (end 52.5 81.5) (width 0.3) (layer "B.Cu") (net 8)))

